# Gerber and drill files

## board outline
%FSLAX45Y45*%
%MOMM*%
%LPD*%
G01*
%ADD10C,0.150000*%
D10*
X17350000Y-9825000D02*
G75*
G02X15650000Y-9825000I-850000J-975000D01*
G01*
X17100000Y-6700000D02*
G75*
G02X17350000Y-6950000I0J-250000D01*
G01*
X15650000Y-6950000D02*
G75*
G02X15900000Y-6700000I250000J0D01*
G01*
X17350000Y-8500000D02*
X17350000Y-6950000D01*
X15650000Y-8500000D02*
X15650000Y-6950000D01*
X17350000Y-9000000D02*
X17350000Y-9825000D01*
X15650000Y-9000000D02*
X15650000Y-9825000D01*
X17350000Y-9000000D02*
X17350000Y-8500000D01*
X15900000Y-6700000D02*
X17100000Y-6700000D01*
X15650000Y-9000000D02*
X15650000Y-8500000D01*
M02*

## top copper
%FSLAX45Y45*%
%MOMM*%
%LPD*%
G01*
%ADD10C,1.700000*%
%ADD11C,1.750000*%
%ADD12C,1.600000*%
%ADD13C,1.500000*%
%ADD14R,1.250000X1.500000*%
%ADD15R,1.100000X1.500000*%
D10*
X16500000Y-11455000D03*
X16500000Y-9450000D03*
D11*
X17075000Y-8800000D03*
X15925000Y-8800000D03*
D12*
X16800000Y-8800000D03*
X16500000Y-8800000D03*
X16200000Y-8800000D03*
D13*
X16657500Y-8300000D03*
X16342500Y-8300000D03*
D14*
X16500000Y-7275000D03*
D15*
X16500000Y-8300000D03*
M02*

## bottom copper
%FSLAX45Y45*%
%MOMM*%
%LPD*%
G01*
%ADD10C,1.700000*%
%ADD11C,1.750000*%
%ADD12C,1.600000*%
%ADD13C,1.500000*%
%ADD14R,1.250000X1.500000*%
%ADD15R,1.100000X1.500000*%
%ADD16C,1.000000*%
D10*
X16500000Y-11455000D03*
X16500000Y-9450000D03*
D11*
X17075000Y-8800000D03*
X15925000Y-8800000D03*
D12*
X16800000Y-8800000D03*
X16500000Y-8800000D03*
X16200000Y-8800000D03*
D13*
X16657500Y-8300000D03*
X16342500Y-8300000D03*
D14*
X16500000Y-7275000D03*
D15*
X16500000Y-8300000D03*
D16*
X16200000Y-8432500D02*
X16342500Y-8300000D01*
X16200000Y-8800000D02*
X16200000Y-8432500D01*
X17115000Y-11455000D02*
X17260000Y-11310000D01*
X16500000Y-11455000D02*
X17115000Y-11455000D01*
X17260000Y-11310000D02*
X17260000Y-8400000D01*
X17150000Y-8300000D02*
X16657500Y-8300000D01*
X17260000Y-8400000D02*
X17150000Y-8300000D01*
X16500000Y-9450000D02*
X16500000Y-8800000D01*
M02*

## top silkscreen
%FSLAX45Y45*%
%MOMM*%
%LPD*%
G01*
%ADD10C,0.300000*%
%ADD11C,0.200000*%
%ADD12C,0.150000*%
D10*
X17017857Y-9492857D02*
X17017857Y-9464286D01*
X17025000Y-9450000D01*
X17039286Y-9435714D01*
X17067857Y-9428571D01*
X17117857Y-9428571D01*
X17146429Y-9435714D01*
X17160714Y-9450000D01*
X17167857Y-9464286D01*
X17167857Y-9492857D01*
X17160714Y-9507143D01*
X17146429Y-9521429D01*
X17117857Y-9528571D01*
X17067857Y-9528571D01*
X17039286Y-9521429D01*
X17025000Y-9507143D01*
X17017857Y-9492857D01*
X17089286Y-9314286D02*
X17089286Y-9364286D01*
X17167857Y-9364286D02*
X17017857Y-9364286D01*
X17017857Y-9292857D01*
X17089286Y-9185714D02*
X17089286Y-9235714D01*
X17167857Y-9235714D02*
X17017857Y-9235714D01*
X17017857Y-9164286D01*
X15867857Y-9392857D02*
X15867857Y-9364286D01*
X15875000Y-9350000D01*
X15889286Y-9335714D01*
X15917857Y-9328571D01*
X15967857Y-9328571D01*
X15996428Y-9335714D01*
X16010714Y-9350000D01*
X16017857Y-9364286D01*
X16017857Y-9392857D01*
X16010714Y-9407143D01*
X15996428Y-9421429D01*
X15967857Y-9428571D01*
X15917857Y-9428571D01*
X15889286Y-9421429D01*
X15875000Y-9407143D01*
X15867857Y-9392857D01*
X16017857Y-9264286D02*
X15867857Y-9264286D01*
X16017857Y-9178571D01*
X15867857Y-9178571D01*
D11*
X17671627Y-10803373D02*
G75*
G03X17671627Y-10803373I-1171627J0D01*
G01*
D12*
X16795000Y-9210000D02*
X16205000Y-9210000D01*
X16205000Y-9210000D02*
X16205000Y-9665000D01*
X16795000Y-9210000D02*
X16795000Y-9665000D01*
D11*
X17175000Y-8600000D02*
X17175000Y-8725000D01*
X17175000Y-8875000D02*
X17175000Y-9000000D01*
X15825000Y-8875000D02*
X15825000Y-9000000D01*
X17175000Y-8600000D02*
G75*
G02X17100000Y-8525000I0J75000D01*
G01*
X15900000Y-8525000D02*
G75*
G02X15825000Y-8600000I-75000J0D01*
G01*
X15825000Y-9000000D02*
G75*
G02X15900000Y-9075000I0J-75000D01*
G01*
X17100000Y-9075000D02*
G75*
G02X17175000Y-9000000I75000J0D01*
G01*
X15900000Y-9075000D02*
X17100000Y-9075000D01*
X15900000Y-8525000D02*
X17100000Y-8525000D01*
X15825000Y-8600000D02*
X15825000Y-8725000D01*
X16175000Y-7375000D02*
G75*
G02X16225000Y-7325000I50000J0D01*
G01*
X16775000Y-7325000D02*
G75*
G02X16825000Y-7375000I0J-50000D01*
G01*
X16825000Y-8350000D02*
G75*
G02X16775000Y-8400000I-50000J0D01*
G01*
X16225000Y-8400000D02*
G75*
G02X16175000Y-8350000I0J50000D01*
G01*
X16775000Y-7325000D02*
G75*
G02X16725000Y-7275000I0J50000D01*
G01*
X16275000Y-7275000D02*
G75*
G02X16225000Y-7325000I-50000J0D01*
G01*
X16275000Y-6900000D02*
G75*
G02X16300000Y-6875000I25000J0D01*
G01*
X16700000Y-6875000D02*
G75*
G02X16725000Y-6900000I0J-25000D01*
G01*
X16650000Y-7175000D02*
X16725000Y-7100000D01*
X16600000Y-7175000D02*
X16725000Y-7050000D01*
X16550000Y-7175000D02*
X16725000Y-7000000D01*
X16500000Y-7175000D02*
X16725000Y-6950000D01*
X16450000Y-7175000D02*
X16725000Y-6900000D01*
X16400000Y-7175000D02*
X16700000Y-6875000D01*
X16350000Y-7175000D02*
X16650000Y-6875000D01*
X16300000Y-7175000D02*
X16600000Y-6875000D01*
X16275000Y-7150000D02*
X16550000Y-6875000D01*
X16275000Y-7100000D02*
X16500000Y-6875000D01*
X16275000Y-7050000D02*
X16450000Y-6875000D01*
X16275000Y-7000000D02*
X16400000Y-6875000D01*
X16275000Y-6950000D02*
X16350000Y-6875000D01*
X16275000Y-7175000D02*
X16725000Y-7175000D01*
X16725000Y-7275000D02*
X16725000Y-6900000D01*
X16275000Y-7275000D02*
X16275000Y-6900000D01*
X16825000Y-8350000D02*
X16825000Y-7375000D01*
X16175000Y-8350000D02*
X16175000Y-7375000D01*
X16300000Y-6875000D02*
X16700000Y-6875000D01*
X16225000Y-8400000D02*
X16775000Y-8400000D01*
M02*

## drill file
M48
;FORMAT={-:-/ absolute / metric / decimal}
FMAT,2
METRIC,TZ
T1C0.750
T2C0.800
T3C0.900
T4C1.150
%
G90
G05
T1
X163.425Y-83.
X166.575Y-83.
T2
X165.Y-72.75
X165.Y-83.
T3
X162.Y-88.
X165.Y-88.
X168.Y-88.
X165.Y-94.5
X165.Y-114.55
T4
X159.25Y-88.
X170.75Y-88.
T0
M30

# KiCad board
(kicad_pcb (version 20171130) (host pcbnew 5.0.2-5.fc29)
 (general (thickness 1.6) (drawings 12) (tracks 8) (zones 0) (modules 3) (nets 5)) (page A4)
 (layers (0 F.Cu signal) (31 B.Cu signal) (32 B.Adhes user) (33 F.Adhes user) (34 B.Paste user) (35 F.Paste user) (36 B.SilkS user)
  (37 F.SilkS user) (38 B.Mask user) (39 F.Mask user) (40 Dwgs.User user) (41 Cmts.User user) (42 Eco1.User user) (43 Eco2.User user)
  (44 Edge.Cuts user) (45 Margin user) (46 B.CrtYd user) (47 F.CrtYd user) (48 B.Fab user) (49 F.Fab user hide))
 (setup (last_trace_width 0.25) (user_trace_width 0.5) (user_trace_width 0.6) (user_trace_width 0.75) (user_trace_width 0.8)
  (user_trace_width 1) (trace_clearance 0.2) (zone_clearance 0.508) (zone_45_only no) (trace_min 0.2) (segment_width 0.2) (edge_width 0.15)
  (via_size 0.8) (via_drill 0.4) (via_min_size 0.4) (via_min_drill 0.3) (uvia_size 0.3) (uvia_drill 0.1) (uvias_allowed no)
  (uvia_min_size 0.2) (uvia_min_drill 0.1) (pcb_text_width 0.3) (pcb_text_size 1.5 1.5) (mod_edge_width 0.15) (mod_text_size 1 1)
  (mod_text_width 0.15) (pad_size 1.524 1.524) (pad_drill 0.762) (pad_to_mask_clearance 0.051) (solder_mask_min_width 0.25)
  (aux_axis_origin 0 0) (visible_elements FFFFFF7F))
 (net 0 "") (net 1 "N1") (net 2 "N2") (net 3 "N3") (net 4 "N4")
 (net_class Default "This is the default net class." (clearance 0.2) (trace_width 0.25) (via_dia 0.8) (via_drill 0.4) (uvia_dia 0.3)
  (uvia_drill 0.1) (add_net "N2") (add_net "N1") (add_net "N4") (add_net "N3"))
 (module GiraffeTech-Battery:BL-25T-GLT (layer F.Cu) (at 165 94.5 270)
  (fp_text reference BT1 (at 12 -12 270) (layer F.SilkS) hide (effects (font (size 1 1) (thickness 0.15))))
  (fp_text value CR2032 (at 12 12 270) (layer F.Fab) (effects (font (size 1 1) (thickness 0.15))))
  (fp_circle (center 13.533734 0) (end 24.007912 5.25) (layer F.SilkS) (width 0.2))
  (fp_line (start -2.4 -2.95) (end -2.4 2.95) (layer F.SilkS) (width 0.15))
  (fp_line (start -2.4 2.95) (end 2.15 2.95) (layer F.SilkS) (width 0.15))
  (fp_line (start -2.4 -2.95) (end 2.15 -2.95) (layer F.SilkS) (width 0.15))
  (pad 2 thru_hole circle (at 20.05 0 270) (size 1.7 1.7) (drill 0.9) (layers *.Cu *.Mask) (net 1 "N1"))
  (pad 1 thru_hole circle (at 0 0 270) (size 1.7 1.7) (drill 0.9) (layers *.Cu *.Mask) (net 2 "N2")))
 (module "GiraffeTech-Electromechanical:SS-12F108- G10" (layer F.Cu) (at 165 88)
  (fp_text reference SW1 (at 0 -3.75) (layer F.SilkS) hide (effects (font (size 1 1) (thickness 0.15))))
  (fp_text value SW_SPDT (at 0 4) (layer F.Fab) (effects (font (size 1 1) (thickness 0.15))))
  (fp_line (start 6.75 -2) (end 6.75 -0.75) (layer F.SilkS) (width 0.2))
  (fp_line (start 6.75 0.75) (end 6.75 2) (layer F.SilkS) (width 0.2))
  (fp_line (start -6.75 0.75) (end -6.75 2) (layer F.SilkS) (width 0.2))
  (fp_arc (start 6.75 -2.75) (end 6 -2.75) (angle -90) (layer F.SilkS) (width 0.2))
  (fp_arc (start -6.75 -2.75) (end -6.75 -2) (angle -90) (layer F.SilkS) (width 0.2))
  (fp_arc (start -6.75 2.75) (end -6 2.75) (angle -90) (layer F.SilkS) (width 0.2))
  (fp_arc (start 6.75 2.75) (end 6.75 2) (angle -90) (layer F.SilkS) (width 0.2))
  (fp_line (start -6 2.75) (end 6 2.75) (layer F.SilkS) (width 0.2))
  (fp_line (start -6 -2.75) (end 6 -2.75) (layer F.SilkS) (width 0.2))
  (fp_line (start -6.75 -2) (end -6.75 -0.75) (layer F.SilkS) (width 0.2))
  (pad MP thru_hole circle (at 5.75 0) (size 1.75 1.75) (drill 1.15) (layers *.Cu *.Mask))
  (pad MP thru_hole circle (at -5.75 0) (size 1.75 1.75) (drill 1.15) (layers *.Cu *.Mask))
  (pad 3 thru_hole circle (at 3 0) (size 1.6 1.6) (drill 0.9) (layers *.Cu *.Mask) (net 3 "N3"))
  (pad 2 thru_hole circle (at 0 0) (size 1.6 1.6) (drill 0.9) (layers *.Cu *.Mask) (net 2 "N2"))
  (pad 1 thru_hole circle (at -3 0) (size 1.6 1.6) (drill 0.9) (layers *.Cu *.Mask) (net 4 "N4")))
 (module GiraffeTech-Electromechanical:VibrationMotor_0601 (layer F.Cu) (at 165 77.5)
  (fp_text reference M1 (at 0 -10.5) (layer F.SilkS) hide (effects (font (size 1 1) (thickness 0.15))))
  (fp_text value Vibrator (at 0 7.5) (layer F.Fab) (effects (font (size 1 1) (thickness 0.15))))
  (fp_arc (start -2.75 -3.75) (end -2.75 -4.25) (angle -90) (layer F.SilkS) (width 0.2))
  (fp_arc (start 2.75 -3.75) (end 3.25 -3.75) (angle -90) (layer F.SilkS) (width 0.2))
  (fp_arc (start 2.75 6) (end 2.75 6.5) (angle -90) (layer F.SilkS) (width 0.2))
  (fp_arc (start -2.75 6) (end -3.25 6) (angle -90) (layer F.SilkS) (width 0.2))
  (fp_arc (start 2.75 -4.75) (end 2.25 -4.75) (angle -90) (layer F.SilkS) (width 0.2))
  (fp_arc (start -2.75 -4.75) (end -2.75 -4.25) (angle -90) (layer F.SilkS) (width 0.2))
  (fp_arc (start -2 -8.5) (end -2 -8.75) (angle -90) (layer F.SilkS) (width 0.2))
  (fp_arc (start 2 -8.5) (end 2.25 -8.5) (angle -90) (layer F.SilkS) (width 0.2))
  (fp_line (start 1.5 -5.75) (end 2.25 -6.5) (layer F.SilkS) (width 0.2))
  (fp_line (start 1 -5.75) (end 2.25 -7) (layer F.SilkS) (width 0.2))
  (fp_line (start 0.5 -5.75) (end 2.25 -7.5) (layer F.SilkS) (width 0.2))
  (fp_line (start 0 -5.75) (end 2.25 -8) (layer F.SilkS) (width 0.2))
  (fp_line (start -0.5 -5.75) (end 2.25 -8.5) (layer F.SilkS) (width 0.2))
  (fp_line (start -1 -5.75) (end 2 -8.75) (layer F.SilkS) (width 0.2))
  (fp_line (start -1.5 -5.75) (end 1.5 -8.75) (layer F.SilkS) (width 0.2))
  (fp_line (start -2 -5.75) (end 1 -8.75) (layer F.SilkS) (width 0.2))
  (fp_line (start -2.25 -6) (end 0.5 -8.75) (layer F.SilkS) (width 0.2))
  (fp_line (start -2.25 -6.5) (end 0 -8.75) (layer F.SilkS) (width 0.2))
  (fp_line (start -2.25 -7) (end -0.5 -8.75) (layer F.SilkS) (width 0.2))
  (fp_line (start -2.25 -7.5) (end -1 -8.75) (layer F.SilkS) (width 0.2))
  (fp_line (start -2.25 -8) (end -1.5 -8.75) (layer F.SilkS) (width 0.2))
  (fp_line (start -2.25 -5.75) (end 2.25 -5.75) (layer F.SilkS) (width 0.2))
  (fp_line (start 2.25 -4.75) (end 2.25 -8.5) (layer F.SilkS) (width 0.2))
  (fp_line (start -2.25 -4.75) (end -2.25 -8.5) (layer F.SilkS) (width 0.2))
  (fp_line (start 3.25 6) (end 3.25 -3.75) (layer F.SilkS) (width 0.2))
  (fp_line (start -3.25 6) (end -3.25 -3.75) (layer F.SilkS) (width 0.2))
  (fp_line (start -2 -8.75) (end 2 -8.75) (layer F.SilkS) (width 0.2))
  (fp_line (start -2.75 6.5) (end 2.75 6.5) (layer F.SilkS) (width 0.2))
  (pad 2 thru_hole circle (at 1.575 5.5) (size 1.5 1.5) (drill 0.75) (layers *.Cu *.Mask) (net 1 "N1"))
  (pad 1 thru_hole circle (at -1.575 5.5) (size 1.5 1.5) (drill 0.75) (layers *.Cu *.Mask) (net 4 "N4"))
  (pad MP thru_hole rect (at 0 -4.75) (size 1.25 1.5) (drill 0.8) (layers *.Cu *.Mask))
  (pad MP thru_hole rect (at 0 5.5) (size 1.1 1.5) (drill 0.8) (layers *.Cu *.Mask)))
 (gr_arc (start 164.999999 107.999999) (end 156.5 98.25) (angle -277.8364977) (layer Edge.Cuts) (width 0.15))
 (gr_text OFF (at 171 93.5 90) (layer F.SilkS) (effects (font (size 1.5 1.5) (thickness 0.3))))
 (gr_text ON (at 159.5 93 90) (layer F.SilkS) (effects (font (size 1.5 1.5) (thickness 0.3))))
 (gr_arc (start 171 69.5) (end 173.5 69.5) (angle -90) (layer Edge.Cuts) (width 0.15))
 (gr_arc (start 159 69.5) (end 159 67) (angle -90) (layer Edge.Cuts) (width 0.15))
 (gr_line (start 173.5 85) (end 173.5 69.5) (layer Edge.Cuts) (width 0.15))
 (gr_line (start 156.5 85) (end 156.5 69.5) (layer Edge.Cuts) (width 0.15))
 (gr_line (start 173.5 90) (end 173.5 98.25) (layer Edge.Cuts) (width 0.15))
 (gr_line (start 156.5 90) (end 156.5 98.25) (layer Edge.Cuts) (width 0.15))
 (gr_line (start 173.5 90) (end 173.5 85) (layer Edge.Cuts) (width 0.15))
 (gr_line (start 159 67) (end 171 67) (layer Edge.Cuts) (width 0.15))
 (gr_line (start 156.5 90) (end 156.5 85) (layer Edge.Cuts) (width 0.15))
 (segment (start 162 84.325) (end 163.425 83) (width 1) (layer B.Cu) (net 4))
 (segment (start 162 88) (end 162 84.325) (width 1) (layer B.Cu) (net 4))
 (segment (start 171.15 114.55) (end 172.6 113.1) (width 1) (layer B.Cu) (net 1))
 (segment (start 165 114.55) (end 171.15 114.55) (width 1) (layer B.Cu) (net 1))
 (segment (start 172.6 113.1) (end 172.6 84) (width 1) (layer B.Cu) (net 1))
 (segment (start 171.5 83) (end 166.575 83) (width 1) (layer B.Cu) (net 1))
 (segment (start 172.6 84) (end 171.5 83) (width 1) (layer B.Cu) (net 1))
 (segment (start 165 94.5) (end 165 88) (width 1) (layer B.Cu) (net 2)))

